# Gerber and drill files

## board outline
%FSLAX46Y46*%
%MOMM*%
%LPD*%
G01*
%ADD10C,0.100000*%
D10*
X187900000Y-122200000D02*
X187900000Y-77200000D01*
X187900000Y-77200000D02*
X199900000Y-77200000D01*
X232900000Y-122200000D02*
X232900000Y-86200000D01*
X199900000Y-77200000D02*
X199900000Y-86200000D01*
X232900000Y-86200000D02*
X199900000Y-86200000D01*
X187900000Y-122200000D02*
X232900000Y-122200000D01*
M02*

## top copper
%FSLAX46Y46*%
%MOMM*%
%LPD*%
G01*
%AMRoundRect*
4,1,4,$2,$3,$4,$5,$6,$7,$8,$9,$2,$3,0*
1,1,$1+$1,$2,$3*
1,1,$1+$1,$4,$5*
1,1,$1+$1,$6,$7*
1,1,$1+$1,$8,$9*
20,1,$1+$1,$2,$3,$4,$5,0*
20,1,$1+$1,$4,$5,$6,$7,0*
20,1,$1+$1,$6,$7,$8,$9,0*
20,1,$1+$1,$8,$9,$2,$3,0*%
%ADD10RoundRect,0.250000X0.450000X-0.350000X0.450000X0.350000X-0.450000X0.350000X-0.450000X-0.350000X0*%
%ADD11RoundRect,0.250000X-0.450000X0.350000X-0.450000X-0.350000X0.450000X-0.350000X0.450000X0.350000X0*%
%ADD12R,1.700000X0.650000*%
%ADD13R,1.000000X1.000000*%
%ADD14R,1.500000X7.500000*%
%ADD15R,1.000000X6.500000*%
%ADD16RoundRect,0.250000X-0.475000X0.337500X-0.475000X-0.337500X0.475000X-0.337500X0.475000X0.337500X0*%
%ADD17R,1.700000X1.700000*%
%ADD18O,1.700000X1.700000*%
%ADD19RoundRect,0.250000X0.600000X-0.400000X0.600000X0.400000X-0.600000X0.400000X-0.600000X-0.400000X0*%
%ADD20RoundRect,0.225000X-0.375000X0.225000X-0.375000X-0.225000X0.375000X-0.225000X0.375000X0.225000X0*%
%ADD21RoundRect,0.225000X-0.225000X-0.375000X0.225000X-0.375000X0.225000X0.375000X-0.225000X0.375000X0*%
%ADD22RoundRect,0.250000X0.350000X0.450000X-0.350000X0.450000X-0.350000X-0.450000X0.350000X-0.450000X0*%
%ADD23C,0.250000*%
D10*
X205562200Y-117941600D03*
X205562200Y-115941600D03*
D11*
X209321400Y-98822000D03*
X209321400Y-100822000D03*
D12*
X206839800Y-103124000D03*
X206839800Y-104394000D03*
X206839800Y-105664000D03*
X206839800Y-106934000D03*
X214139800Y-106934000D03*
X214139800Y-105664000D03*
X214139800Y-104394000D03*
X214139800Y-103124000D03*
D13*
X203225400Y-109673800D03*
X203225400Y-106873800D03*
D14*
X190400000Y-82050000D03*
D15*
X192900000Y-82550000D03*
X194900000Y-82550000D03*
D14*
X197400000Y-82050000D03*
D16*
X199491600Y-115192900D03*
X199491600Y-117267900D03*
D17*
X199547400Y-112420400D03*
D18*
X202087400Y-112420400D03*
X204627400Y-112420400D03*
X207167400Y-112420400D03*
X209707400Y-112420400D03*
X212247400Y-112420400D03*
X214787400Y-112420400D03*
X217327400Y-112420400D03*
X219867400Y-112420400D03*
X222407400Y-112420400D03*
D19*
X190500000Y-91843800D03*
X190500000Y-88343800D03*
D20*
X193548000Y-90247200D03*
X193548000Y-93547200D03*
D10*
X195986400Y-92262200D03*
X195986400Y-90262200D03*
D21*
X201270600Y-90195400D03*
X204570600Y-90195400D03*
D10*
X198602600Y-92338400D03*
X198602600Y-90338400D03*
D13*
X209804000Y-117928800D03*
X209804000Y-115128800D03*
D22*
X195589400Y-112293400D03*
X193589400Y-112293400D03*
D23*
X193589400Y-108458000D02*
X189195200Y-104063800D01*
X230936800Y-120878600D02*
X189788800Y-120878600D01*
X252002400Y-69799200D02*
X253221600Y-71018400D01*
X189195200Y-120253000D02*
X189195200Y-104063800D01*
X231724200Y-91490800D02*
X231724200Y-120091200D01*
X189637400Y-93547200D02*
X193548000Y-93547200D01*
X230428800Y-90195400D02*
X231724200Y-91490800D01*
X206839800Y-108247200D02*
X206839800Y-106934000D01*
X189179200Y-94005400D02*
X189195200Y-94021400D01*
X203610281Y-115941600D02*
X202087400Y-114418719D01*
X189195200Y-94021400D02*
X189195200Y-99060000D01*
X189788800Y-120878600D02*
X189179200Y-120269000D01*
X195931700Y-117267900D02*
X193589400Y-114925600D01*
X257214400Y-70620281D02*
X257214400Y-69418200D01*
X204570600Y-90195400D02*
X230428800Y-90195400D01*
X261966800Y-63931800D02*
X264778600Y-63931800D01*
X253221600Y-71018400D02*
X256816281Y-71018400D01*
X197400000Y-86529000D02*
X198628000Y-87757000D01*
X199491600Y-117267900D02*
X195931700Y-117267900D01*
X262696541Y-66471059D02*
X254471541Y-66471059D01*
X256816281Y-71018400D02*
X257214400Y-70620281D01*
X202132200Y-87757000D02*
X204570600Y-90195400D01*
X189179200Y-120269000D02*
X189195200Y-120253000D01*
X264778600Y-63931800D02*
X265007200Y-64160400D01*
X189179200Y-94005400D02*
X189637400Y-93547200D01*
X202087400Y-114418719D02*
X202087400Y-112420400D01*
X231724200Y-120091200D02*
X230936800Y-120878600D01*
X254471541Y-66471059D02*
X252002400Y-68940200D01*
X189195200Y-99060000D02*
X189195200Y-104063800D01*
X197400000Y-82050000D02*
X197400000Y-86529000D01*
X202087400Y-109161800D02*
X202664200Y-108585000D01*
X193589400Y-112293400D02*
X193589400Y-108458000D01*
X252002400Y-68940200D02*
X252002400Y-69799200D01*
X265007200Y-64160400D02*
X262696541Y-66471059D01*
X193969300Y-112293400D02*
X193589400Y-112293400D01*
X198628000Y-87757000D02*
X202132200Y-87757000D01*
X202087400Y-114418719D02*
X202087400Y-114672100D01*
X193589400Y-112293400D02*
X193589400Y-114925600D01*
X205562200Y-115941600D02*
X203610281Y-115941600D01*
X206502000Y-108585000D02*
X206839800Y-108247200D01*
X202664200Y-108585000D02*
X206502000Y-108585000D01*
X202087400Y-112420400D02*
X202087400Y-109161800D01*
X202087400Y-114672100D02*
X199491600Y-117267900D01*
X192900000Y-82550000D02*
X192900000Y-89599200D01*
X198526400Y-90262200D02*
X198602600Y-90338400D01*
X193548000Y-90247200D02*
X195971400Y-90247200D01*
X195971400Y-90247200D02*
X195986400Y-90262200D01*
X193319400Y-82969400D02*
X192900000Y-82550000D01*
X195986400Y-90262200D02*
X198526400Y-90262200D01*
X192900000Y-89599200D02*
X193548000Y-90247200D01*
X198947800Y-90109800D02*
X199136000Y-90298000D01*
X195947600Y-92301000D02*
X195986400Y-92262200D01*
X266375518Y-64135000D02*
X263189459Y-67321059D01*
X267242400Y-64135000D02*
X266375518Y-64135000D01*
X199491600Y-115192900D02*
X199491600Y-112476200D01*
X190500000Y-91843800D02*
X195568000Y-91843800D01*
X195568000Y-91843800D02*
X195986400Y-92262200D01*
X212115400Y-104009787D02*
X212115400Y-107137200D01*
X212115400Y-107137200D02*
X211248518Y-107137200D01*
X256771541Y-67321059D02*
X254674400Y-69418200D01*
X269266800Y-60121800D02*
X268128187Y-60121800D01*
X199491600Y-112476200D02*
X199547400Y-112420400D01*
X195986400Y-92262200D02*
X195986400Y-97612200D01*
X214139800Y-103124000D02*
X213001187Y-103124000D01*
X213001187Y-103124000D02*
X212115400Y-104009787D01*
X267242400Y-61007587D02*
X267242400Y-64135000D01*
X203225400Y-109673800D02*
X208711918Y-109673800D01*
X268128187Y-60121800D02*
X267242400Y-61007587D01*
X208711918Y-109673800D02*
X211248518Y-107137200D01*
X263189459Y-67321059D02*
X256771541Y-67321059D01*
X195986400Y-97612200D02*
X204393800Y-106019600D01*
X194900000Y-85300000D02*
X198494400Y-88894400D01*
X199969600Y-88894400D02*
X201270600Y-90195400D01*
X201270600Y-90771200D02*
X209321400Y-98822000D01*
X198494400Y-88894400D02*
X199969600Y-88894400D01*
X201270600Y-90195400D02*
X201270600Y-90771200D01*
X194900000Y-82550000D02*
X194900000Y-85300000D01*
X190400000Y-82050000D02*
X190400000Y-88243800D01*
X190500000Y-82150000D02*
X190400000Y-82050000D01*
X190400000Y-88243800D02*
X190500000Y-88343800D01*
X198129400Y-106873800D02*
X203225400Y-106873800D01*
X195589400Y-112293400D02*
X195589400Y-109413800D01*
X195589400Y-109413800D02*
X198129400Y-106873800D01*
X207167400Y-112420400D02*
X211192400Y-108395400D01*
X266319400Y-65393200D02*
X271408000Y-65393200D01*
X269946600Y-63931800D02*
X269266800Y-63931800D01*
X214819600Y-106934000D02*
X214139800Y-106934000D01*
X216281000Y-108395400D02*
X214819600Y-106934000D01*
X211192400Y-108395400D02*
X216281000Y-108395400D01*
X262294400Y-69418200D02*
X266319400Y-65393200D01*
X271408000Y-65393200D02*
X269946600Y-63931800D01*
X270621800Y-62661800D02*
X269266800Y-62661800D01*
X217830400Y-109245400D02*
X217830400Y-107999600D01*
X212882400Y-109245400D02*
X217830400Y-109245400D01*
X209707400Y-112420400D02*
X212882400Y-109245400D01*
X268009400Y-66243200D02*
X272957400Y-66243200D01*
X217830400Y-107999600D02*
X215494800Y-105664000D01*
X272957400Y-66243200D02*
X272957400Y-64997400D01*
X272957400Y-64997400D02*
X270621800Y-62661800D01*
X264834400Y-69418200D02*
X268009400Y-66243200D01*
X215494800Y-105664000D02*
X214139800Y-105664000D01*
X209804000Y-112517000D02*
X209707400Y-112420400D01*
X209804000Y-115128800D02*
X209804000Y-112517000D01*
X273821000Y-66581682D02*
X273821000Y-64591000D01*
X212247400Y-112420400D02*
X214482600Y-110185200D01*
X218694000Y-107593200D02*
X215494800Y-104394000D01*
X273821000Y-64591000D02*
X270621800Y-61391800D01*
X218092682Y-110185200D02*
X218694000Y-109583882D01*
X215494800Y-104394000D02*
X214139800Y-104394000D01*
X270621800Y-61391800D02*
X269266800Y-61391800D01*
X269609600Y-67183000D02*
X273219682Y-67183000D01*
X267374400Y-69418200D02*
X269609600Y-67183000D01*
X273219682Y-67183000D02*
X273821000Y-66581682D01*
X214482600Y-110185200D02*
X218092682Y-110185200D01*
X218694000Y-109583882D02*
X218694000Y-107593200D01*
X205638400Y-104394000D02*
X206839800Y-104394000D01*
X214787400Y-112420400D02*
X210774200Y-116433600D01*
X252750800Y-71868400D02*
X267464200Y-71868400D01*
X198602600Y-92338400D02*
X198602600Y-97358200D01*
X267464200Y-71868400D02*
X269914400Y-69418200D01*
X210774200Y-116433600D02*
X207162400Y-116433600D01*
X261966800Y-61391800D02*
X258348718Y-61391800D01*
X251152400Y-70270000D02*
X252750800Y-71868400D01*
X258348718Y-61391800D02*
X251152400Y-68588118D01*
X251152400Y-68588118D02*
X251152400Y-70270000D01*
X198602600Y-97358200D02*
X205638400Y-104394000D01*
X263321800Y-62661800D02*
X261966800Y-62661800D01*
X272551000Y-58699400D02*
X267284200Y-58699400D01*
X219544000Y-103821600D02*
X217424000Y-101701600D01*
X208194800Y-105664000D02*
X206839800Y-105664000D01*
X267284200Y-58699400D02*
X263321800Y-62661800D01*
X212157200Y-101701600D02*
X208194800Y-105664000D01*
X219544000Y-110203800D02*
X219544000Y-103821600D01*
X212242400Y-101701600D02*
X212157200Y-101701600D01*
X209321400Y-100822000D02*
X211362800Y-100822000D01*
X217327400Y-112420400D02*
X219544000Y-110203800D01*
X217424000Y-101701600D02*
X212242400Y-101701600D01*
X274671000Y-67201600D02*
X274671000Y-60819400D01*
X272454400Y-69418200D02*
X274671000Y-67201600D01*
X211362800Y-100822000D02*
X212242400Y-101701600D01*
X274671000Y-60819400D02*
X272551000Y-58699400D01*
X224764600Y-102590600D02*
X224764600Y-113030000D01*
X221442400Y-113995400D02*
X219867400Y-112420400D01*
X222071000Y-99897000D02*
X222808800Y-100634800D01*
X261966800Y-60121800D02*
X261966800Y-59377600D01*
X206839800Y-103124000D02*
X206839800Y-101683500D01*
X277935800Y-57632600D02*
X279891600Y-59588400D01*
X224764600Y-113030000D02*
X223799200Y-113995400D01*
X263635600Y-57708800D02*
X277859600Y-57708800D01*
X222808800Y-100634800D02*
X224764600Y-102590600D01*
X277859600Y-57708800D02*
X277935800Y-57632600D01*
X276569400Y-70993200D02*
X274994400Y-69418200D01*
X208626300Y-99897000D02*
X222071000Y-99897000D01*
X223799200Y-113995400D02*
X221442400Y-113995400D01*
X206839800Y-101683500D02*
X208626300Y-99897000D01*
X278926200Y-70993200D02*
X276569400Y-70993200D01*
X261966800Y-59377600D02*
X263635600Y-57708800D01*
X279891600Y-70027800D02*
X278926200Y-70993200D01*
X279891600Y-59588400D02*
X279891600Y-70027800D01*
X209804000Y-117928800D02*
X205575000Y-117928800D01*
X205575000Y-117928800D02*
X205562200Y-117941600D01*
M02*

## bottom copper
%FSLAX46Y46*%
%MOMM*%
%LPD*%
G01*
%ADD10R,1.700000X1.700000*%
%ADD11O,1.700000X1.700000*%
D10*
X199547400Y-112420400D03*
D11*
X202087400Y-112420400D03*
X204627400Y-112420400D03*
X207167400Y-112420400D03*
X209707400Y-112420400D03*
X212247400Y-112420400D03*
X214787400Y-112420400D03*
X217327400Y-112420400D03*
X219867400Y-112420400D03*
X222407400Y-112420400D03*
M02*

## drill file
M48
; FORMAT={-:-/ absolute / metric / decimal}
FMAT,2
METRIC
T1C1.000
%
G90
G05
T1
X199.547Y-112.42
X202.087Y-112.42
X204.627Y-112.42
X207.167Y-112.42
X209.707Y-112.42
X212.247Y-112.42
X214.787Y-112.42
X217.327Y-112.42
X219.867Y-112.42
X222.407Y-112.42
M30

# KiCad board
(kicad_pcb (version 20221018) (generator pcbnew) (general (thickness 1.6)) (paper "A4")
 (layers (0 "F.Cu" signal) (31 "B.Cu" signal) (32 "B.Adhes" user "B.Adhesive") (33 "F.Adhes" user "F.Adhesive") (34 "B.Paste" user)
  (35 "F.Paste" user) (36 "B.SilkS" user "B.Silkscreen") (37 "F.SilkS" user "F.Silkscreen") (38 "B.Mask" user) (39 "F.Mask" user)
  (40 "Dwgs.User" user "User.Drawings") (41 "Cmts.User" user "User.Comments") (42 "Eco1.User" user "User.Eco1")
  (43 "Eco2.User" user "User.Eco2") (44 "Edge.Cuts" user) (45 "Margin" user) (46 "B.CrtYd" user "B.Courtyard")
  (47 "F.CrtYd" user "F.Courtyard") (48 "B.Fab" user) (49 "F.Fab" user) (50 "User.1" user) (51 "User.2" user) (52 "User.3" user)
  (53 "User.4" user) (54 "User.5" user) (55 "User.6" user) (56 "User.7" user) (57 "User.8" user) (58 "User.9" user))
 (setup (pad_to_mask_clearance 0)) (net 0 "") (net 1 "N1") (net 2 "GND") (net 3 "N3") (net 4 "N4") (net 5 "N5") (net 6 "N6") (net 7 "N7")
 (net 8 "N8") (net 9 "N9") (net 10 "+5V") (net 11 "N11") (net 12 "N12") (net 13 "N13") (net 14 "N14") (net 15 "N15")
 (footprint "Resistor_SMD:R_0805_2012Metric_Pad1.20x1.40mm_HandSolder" (layer "F.Cu") (at 205.5622 116.9416 90)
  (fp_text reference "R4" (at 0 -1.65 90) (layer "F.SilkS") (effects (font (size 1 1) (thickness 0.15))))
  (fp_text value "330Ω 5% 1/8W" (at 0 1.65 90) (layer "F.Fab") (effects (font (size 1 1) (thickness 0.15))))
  (pad "1" smd roundrect (at -1 0 90) (size 1.2 1.4) (layers "F.Cu" "F.Paste" "F.Mask") (roundrect_rratio 0.208333) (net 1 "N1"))
  (pad "2" smd roundrect (at 1 0 90) (size 1.2 1.4) (layers "F.Cu" "F.Paste" "F.Mask") (roundrect_rratio 0.208333) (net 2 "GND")))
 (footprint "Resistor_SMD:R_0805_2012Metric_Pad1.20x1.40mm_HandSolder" (layer "F.Cu") (at 209.3214 99.822 -90)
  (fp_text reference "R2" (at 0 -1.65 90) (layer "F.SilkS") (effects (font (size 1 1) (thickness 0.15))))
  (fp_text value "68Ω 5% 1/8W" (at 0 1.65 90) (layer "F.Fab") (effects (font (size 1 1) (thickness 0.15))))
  (pad "1" smd roundrect (at -1 0 270) (size 1.2 1.4) (layers "F.Cu" "F.Paste" "F.Mask") (roundrect_rratio 0.208333) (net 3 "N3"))
  (pad "2" smd roundrect (at 1 0 270) (size 1.2 1.4) (layers "F.Cu" "F.Paste" "F.Mask") (roundrect_rratio 0.208333) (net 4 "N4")))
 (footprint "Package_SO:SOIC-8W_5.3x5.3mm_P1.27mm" (layer "F.Cu") (at 210.4898 105.029)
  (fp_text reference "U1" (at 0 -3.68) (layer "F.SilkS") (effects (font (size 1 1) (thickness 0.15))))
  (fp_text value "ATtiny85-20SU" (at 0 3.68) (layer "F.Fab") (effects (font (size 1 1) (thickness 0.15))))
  (pad "1" smd rect (at -3.65 -1.905) (size 1.7 0.65) (layers "F.Cu" "F.Paste" "F.Mask") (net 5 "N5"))
  (pad "2" smd rect (at -3.65 -0.635) (size 1.7 0.65) (layers "F.Cu" "F.Paste" "F.Mask") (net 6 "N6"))
  (pad "3" smd rect (at -3.65 0.635) (size 1.7 0.65) (layers "F.Cu" "F.Paste" "F.Mask") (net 4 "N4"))
  (pad "4" smd rect (at -3.65 1.905) (size 1.7 0.65) (layers "F.Cu" "F.Paste" "F.Mask") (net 2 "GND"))
  (pad "5" smd rect (at 3.65 1.905) (size 1.7 0.65) (layers "F.Cu" "F.Paste" "F.Mask") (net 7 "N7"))
  (pad "6" smd rect (at 3.65 0.635) (size 1.7 0.65) (layers "F.Cu" "F.Paste" "F.Mask") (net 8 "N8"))
  (pad "7" smd rect (at 3.65 -0.635) (size 1.7 0.65) (layers "F.Cu" "F.Paste" "F.Mask") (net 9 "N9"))
  (pad "8" smd rect (at 3.65 -1.905) (size 1.7 0.65) (layers "F.Cu" "F.Paste" "F.Mask") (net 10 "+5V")))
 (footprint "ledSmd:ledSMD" (layer "F.Cu") (at 203.2254 107.8738 90)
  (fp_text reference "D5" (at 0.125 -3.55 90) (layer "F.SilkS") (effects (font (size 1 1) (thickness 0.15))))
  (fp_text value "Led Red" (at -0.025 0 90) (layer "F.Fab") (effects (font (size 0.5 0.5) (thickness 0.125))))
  (pad "1" smd rect (at -1.8 0 90) (size 1 1) (layers "F.Cu" "F.Paste" "F.Mask") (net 10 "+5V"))
  (pad "2" smd rect (at 1 0 90) (size 1 1) (layers "F.Cu" "F.Paste" "F.Mask") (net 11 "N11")))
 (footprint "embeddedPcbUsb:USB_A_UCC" (layer "F.Cu") (at 193.9 82.25 -90)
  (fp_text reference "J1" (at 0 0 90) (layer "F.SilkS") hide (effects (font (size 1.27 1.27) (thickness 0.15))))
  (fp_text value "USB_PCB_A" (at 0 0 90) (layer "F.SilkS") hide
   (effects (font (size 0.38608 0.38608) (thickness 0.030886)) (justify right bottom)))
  (pad "1" smd rect (at -0.2 3.5 270) (size 7.5 1.5) (layers "F.Cu" "F.Paste" "F.Mask") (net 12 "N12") (solder_mask_margin 0.1016))
  (pad "2" smd rect (at 0.3 1 270) (size 6.5 1) (layers "F.Cu" "F.Paste" "F.Mask") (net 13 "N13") (solder_mask_margin 0.1016))
  (pad "3" smd rect (at 0.3 -1 270) (size 6.5 1) (layers "F.Cu" "F.Paste" "F.Mask") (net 3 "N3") (solder_mask_margin 0.1016))
  (pad "4" smd rect (at -0.2 -3.5 270) (size 7.5 1.5) (layers "F.Cu" "F.Paste" "F.Mask") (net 2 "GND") (solder_mask_margin 0.1016)))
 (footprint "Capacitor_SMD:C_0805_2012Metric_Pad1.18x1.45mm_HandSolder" (layer "F.Cu") (at 199.4916 116.2304 -90)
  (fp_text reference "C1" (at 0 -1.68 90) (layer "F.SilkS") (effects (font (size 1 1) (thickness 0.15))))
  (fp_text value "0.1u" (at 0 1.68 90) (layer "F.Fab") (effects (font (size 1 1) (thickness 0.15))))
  (pad "1" smd roundrect (at -1.0375 0 270) (size 1.175 1.45) (layers "F.Cu" "F.Paste" "F.Mask") (roundrect_rratio 0.212766) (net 10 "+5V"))
  (pad "2" smd roundrect (at 1.0375 0 270) (size 1.175 1.45) (layers "F.Cu" "F.Paste" "F.Mask") (roundrect_rratio 0.212766) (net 2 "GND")))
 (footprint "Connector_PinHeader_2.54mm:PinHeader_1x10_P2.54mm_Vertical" (layer "F.Cu") (at 199.5474 112.4204 90)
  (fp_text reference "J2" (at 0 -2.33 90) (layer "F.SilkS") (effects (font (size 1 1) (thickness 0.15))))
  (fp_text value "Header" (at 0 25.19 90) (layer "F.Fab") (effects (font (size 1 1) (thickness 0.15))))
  (pad "1" thru_hole rect (at 0 0 90) (size 1.7 1.7) (drill 1) (layers "*.Cu" "*.Mask") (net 10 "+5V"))
  (pad "2" thru_hole oval (at 0 2.54 90) (size 1.7 1.7) (drill 1) (layers "*.Cu" "*.Mask") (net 2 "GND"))
  (pad "3" thru_hole oval (at 0 5.08 90) (size 1.7 1.7) (drill 1) (layers "*.Cu" "*.Mask") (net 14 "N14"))
  (pad "4" thru_hole oval (at 0 7.62 90) (size 1.7 1.7) (drill 1) (layers "*.Cu" "*.Mask") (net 7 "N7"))
  (pad "5" thru_hole oval (at 0 10.16 90) (size 1.7 1.7) (drill 1) (layers "*.Cu" "*.Mask") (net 8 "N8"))
  (pad "6" thru_hole oval (at 0 12.7 90) (size 1.7 1.7) (drill 1) (layers "*.Cu" "*.Mask") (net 9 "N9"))
  (pad "7" thru_hole oval (at 0 15.24 90) (size 1.7 1.7) (drill 1) (layers "*.Cu" "*.Mask") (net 6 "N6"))
  (pad "8" thru_hole oval (at 0 17.78 90) (size 1.7 1.7) (drill 1) (layers "*.Cu" "*.Mask") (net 4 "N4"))
  (pad "9" thru_hole oval (at 0 20.32 90) (size 1.7 1.7) (drill 1) (layers "*.Cu" "*.Mask") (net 5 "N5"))
  (pad "10" thru_hole oval (at 0 22.86 90) (size 1.7 1.7) (drill 1) (layers "*.Cu" "*.Mask") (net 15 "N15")))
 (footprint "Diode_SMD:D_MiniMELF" (layer "F.Cu") (at 190.5 90.0938 90)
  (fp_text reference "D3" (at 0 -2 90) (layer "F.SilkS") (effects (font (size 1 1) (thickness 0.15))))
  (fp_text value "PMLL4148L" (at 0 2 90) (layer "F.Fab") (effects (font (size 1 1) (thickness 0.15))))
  (pad "1" smd roundrect (at -1.75 0 90) (size 1.3 1.7) (layers "F.Cu" "F.Paste" "F.Mask") (roundrect_rratio 0.1923076923) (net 10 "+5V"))
  (pad "2" smd roundrect (at 1.75 0 90) (size 1.3 1.7) (layers "F.Cu" "F.Paste" "F.Mask") (roundrect_rratio 0.1923076923) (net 12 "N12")))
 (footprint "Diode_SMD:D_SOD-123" (layer "F.Cu") (at 193.548 91.8972 -90)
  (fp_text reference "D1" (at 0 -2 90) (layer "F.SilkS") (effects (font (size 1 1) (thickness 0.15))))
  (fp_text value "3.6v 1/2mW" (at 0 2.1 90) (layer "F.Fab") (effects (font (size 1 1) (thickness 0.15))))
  (pad "1" smd roundrect (at -1.65 0 270) (size 0.9 1.2) (layers "F.Cu" "F.Paste" "F.Mask") (roundrect_rratio 0.25) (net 13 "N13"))
  (pad "2" smd roundrect (at 1.65 0 270) (size 0.9 1.2) (layers "F.Cu" "F.Paste" "F.Mask") (roundrect_rratio 0.25) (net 2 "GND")))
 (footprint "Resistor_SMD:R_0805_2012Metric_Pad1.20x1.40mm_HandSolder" (layer "F.Cu") (at 195.9864 91.2622 90)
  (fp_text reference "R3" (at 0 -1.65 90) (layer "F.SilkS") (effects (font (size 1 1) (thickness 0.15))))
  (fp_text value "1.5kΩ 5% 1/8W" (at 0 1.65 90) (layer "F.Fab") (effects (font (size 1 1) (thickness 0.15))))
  (pad "1" smd roundrect (at -1 0 90) (size 1.2 1.4) (layers "F.Cu" "F.Paste" "F.Mask") (roundrect_rratio 0.208333) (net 10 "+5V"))
  (pad "2" smd roundrect (at 1 0 90) (size 1.2 1.4) (layers "F.Cu" "F.Paste" "F.Mask") (roundrect_rratio 0.208333) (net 13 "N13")))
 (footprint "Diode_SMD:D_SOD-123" (layer "F.Cu") (at 202.9206 90.1954)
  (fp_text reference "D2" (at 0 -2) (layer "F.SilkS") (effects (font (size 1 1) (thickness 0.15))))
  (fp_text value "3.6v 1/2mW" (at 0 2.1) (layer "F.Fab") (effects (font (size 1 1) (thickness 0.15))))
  (pad "1" smd roundrect (at -1.65 0) (size 0.9 1.2) (layers "F.Cu" "F.Paste" "F.Mask") (roundrect_rratio 0.25) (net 3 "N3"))
  (pad "2" smd roundrect (at 1.65 0) (size 0.9 1.2) (layers "F.Cu" "F.Paste" "F.Mask") (roundrect_rratio 0.25) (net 2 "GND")))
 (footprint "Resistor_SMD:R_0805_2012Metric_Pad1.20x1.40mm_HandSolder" (layer "F.Cu") (at 198.6026 91.3384 90)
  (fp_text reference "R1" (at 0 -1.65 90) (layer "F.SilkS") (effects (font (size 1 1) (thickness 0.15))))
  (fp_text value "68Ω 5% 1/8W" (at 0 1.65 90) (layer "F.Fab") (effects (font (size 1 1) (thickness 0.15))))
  (pad "1" smd roundrect (at -1 0 90) (size 1.2 1.4) (layers "F.Cu" "F.Paste" "F.Mask") (roundrect_rratio 0.208333) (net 6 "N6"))
  (pad "2" smd roundrect (at 1 0 90) (size 1.2 1.4) (layers "F.Cu" "F.Paste" "F.Mask") (roundrect_rratio 0.208333) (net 13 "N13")))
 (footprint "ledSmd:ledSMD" (layer "F.Cu") (at 209.804 116.1288 90)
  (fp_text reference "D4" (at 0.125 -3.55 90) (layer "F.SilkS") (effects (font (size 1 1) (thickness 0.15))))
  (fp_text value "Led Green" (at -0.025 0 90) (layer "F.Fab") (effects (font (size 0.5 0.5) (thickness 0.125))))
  (pad "1" smd rect (at -1.8 0 90) (size 1 1) (layers "F.Cu" "F.Paste" "F.Mask") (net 1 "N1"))
  (pad "2" smd rect (at 1 0 90) (size 1 1) (layers "F.Cu" "F.Paste" "F.Mask") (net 8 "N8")))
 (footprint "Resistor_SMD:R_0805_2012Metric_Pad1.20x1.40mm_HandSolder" (layer "F.Cu") (at 194.5894 112.2934 180)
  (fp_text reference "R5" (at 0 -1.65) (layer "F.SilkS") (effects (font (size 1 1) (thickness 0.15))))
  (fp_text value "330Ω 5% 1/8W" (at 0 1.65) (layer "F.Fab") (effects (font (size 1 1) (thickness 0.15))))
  (pad "1" smd roundrect (at -1 0 180) (size 1.2 1.4) (layers "F.Cu" "F.Paste" "F.Mask") (roundrect_rratio 0.208333) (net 11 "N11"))
  (pad "2" smd roundrect (at 1 0 180) (size 1.2 1.4) (layers "F.Cu" "F.Paste" "F.Mask") (roundrect_rratio 0.208333) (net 2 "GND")))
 (gr_line (start 187.9 122.2) (end 187.9 77.2) (stroke (width 0.1) (type default)) (layer "Edge.Cuts"))
 (gr_line (start 187.9 77.2) (end 199.9 77.2) (stroke (width 0.1) (type default)) (layer "Edge.Cuts"))
 (gr_line (start 232.9 122.2) (end 232.9 86.2) (stroke (width 0.1) (type default)) (layer "Edge.Cuts"))
 (gr_line (start 199.9 77.2) (end 199.9 86.2) (stroke (width 0.1) (type default)) (layer "Edge.Cuts"))
 (gr_line (start 232.9 86.2) (end 199.9 86.2) (stroke (width 0.1) (type default)) (layer "Edge.Cuts"))
 (gr_line (start 187.9 122.2) (end 232.9 122.2) (stroke (width 0.1) (type default)) (layer "Edge.Cuts"))
 (segment (start 193.5894 108.458) (end 189.1952 104.0638) (width 0.25) (layer "F.Cu") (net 2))
 (segment (start 230.9368 120.8786) (end 189.7888 120.8786) (width 0.25) (layer "F.Cu") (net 2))
 (segment (start 252.0024 69.7992) (end 253.2216 71.0184) (width 0.25) (layer "F.Cu") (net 2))
 (segment (start 189.1952 120.253) (end 189.1952 104.0638) (width 0.25) (layer "F.Cu") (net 2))
 (segment (start 231.7242 91.4908) (end 231.7242 120.0912) (width 0.25) (layer "F.Cu") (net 2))
 (segment (start 189.6374 93.5472) (end 193.548 93.5472) (width 0.25) (layer "F.Cu") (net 2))
 (segment (start 230.4288 90.1954) (end 231.7242 91.4908) (width 0.25) (layer "F.Cu") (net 2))
 (segment (start 206.8398 108.2472) (end 206.8398 106.934) (width 0.25) (layer "F.Cu") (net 2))
 (segment (start 189.1792 94.0054) (end 189.1952 94.0214) (width 0.25) (layer "F.Cu") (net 2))
 (segment (start 203.610281 115.9416) (end 202.0874 114.418719) (width 0.25) (layer "F.Cu") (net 2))
 (segment (start 189.1952 94.0214) (end 189.1952 99.06) (width 0.25) (layer "F.Cu") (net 2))
 (segment (start 189.7888 120.8786) (end 189.1792 120.269) (width 0.25) (layer "F.Cu") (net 2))
 (segment (start 195.9317 117.2679) (end 193.5894 114.9256) (width 0.25) (layer "F.Cu") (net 2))
 (segment (start 257.2144 70.620281) (end 257.2144 69.4182) (width 0.25) (layer "F.Cu") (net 2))
 (segment (start 204.5706 90.1954) (end 230.4288 90.1954) (width 0.25) (layer "F.Cu") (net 2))
 (segment (start 261.9668 63.9318) (end 264.7786 63.9318) (width 0.25) (layer "F.Cu") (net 2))
 (segment (start 253.2216 71.0184) (end 256.816281 71.0184) (width 0.25) (layer "F.Cu") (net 2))
 (segment (start 197.4 86.529) (end 198.628 87.757) (width 0.25) (layer "F.Cu") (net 2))
 (segment (start 199.4916 117.2679) (end 195.9317 117.2679) (width 0.25) (layer "F.Cu") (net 2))
 (segment (start 262.696541 66.471059) (end 254.471541 66.471059) (width 0.25) (layer "F.Cu") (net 2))
 (segment (start 256.816281 71.0184) (end 257.2144 70.620281) (width 0.25) (layer "F.Cu") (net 2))
 (segment (start 202.1322 87.757) (end 204.5706 90.1954) (width 0.25) (layer "F.Cu") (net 2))
 (segment (start 189.1792 120.269) (end 189.1952 120.253) (width 0.25) (layer "F.Cu") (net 2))
 (segment (start 264.7786 63.9318) (end 265.0072 64.1604) (width 0.25) (layer "F.Cu") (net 2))
 (segment (start 189.1792 94.0054) (end 189.6374 93.5472) (width 0.25) (layer "F.Cu") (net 2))
 (segment (start 202.0874 114.418719) (end 202.0874 112.4204) (width 0.25) (layer "F.Cu") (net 2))
 (segment (start 231.7242 120.0912) (end 230.9368 120.8786) (width 0.25) (layer "F.Cu") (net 2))
 (segment (start 254.471541 66.471059) (end 252.0024 68.9402) (width 0.25) (layer "F.Cu") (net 2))
 (segment (start 189.1952 99.06) (end 189.1952 104.0638) (width 0.25) (layer "F.Cu") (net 2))
 (segment (start 197.4 82.05) (end 197.4 86.529) (width 0.25) (layer "F.Cu") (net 2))
 (segment (start 202.0874 109.1618) (end 202.6642 108.585) (width 0.25) (layer "F.Cu") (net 2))
 (segment (start 193.5894 112.2934) (end 193.5894 108.458) (width 0.25) (layer "F.Cu") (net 2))
 (segment (start 252.0024 68.9402) (end 252.0024 69.7992) (width 0.25) (layer "F.Cu") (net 2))
 (segment (start 265.0072 64.1604) (end 262.696541 66.471059) (width 0.25) (layer "F.Cu") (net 2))
 (segment (start 193.9693 112.2934) (end 193.5894 112.2934) (width 0.25) (layer "F.Cu") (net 2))
 (segment (start 198.628 87.757) (end 202.1322 87.757) (width 0.25) (layer "F.Cu") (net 2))
 (segment (start 202.0874 114.418719) (end 202.0874 114.6721) (width 0.25) (layer "F.Cu") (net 2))
 (segment (start 193.5894 112.2934) (end 193.5894 114.9256) (width 0.25) (layer "F.Cu") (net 2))
 (segment (start 205.5622 115.9416) (end 203.610281 115.9416) (width 0.25) (layer "F.Cu") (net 2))
 (segment (start 206.502 108.585) (end 206.8398 108.2472) (width 0.25) (layer "F.Cu") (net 2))
 (segment (start 202.6642 108.585) (end 206.502 108.585) (width 0.25) (layer "F.Cu") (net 2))
 (segment (start 202.0874 112.4204) (end 202.0874 109.1618) (width 0.25) (layer "F.Cu") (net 2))
 (segment (start 202.0874 114.6721) (end 199.4916 117.2679) (width 0.25) (layer "F.Cu") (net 2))
 (segment (start 192.9 82.55) (end 192.9 89.5992) (width 0.25) (layer "F.Cu") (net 13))
 (segment (start 198.5264 90.2622) (end 198.6026 90.3384) (width 0.25) (layer "F.Cu") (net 13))
 (segment (start 193.548 90.2472) (end 195.9714 90.2472) (width 0.25) (layer "F.Cu") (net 13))
 (segment (start 195.9714 90.2472) (end 195.9864 90.2622) (width 0.25) (layer "F.Cu") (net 13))
 (segment (start 193.3194 82.9694) (end 192.9 82.55) (width 0.25) (layer "F.Cu") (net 13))
 (segment (start 195.9864 90.2622) (end 198.5264 90.2622) (width 0.25) (layer "F.Cu") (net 13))
 (segment (start 192.9 89.5992) (end 193.548 90.2472) (width 0.25) (layer "F.Cu") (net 13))
 (segment (start 198.9478 90.1098) (end 199.136 90.298) (width 0.25) (layer "F.Cu") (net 13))
 (segment (start 195.9476 92.301) (end 195.9864 92.2622) (width 0.25) (layer "F.Cu") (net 10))
 (segment (start 266.375518 64.135) (end 263.189459 67.321059) (width 0.25) (layer "F.Cu") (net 10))
 (segment (start 267.2424 64.135) (end 266.375518 64.135) (width 0.25) (layer "F.Cu") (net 10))
 (segment (start 199.4916 115.1929) (end 199.4916 112.4762) (width 0.25) (layer "F.Cu") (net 10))
 (segment (start 190.5 91.8438) (end 195.568 91.8438) (width 0.25) (layer "F.Cu") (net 10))
 (segment (start 195.568 91.8438) (end 195.9864 92.2622) (width 0.25) (layer "F.Cu") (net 10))
 (segment (start 212.1154 104.009787) (end 212.1154 107.1372) (width 0.25) (layer "F.Cu") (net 10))
 (segment (start 212.1154 107.1372) (end 211.248518 107.1372) (width 0.25) (layer "F.Cu") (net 10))
 (segment (start 256.771541 67.321059) (end 254.6744 69.4182) (width 0.25) (layer "F.Cu") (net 10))
 (segment (start 269.2668 60.1218) (end 268.128187 60.1218) (width 0.25) (layer "F.Cu") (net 10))
 (segment (start 199.4916 112.4762) (end 199.5474 112.4204) (width 0.25) (layer "F.Cu") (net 10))
 (segment (start 195.9864 92.2622) (end 195.9864 97.6122) (width 0.25) (layer "F.Cu") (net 10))
 (segment (start 214.1398 103.124) (end 213.001187 103.124) (width 0.25) (layer "F.Cu") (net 10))
 (segment (start 213.001187 103.124) (end 212.1154 104.009787) (width 0.25) (layer "F.Cu") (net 10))
 (segment (start 267.2424 61.007587) (end 267.2424 64.135) (width 0.25) (layer "F.Cu") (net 10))
 (segment (start 203.2254 109.6738) (end 208.711918 109.6738) (width 0.25) (layer "F.Cu") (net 10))
 (segment (start 268.128187 60.1218) (end 267.2424 61.007587) (width 0.25) (layer "F.Cu") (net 10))
 (segment (start 208.711918 109.6738) (end 211.248518 107.1372) (width 0.25) (layer "F.Cu") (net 10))
 (segment (start 263.189459 67.321059) (end 256.771541 67.321059) (width 0.25) (layer "F.Cu") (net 10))
 (segment (start 195.9864 97.6122) (end 204.3938 106.0196) (width 0.25) (layer "F.Cu") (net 10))
 (segment (start 194.9 85.3) (end 198.4944 88.8944) (width 0.25) (layer "F.Cu") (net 3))
 (segment (start 199.9696 88.8944) (end 201.2706 90.1954) (width 0.25) (layer "F.Cu") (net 3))
 (segment (start 201.2706 90.7712) (end 209.3214 98.822) (width 0.25) (layer "F.Cu") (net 3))
 (segment (start 198.4944 88.8944) (end 199.9696 88.8944) (width 0.25) (layer "F.Cu") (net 3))
 (segment (start 201.2706 90.1954) (end 201.2706 90.7712) (width 0.25) (layer "F.Cu") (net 3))
 (segment (start 194.9 82.55) (end 194.9 85.3) (width 0.25) (layer "F.Cu") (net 3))
 (segment (start 190.4 82.05) (end 190.4 88.2438) (width 0.25) (layer "F.Cu") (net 12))
 (segment (start 190.5 82.15) (end 190.4 82.05) (width 0.25) (layer "F.Cu") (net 12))
 (segment (start 190.4 88.2438) (end 190.5 88.3438) (width 0.25) (layer "F.Cu") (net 12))
 (segment (start 198.1294 106.8738) (end 203.2254 106.8738) (width 0.25) (layer "F.Cu") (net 11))
 (segment (start 195.5894 112.2934) (end 195.5894 109.4138) (width 0.25) (layer "F.Cu") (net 11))
 (segment (start 195.5894 109.4138) (end 198.1294 106.8738) (width 0.25) (layer "F.Cu") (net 11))
 (segment (start 207.1674 112.4204) (end 211.1924 108.3954) (width 0.25) (layer "F.Cu") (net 7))
 (segment (start 266.3194 65.3932) (end 271.408 65.3932) (width 0.25) (layer "F.Cu") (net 7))
 (segment (start 269.9466 63.9318) (end 269.2668 63.9318) (width 0.25) (layer "F.Cu") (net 7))
 (segment (start 214.8196 106.934) (end 214.1398 106.934) (width 0.25) (layer "F.Cu") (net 7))
 (segment (start 216.281 108.3954) (end 214.8196 106.934) (width 0.25) (layer "F.Cu") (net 7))
 (segment (start 211.1924 108.3954) (end 216.281 108.3954) (width 0.25) (layer "F.Cu") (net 7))
 (segment (start 262.2944 69.4182) (end 266.3194 65.3932) (width 0.25) (layer "F.Cu") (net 7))
 (segment (start 271.408 65.3932) (end 269.9466 63.9318) (width 0.25) (layer "F.Cu") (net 7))
 (segment (start 270.6218 62.6618) (end 269.2668 62.6618) (width 0.25) (layer "F.Cu") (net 8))
 (segment (start 217.8304 109.2454) (end 217.8304 107.9996) (width 0.25) (layer "F.Cu") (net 8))
 (segment (start 212.8824 109.2454) (end 217.8304 109.2454) (width 0.25) (layer "F.Cu") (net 8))
 (segment (start 209.7074 112.4204) (end 212.8824 109.2454) (width 0.25) (layer "F.Cu") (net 8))
 (segment (start 268.0094 66.2432) (end 272.9574 66.2432) (width 0.25) (layer "F.Cu") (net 8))
 (segment (start 217.8304 107.9996) (end 215.4948 105.664) (width 0.25) (layer "F.Cu") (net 8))
 (segment (start 272.9574 66.2432) (end 272.9574 64.9974) (width 0.25) (layer "F.Cu") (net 8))
 (segment (start 272.9574 64.9974) (end 270.6218 62.6618) (width 0.25) (layer "F.Cu") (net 8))
 (segment (start 264.8344 69.4182) (end 268.0094 66.2432) (width 0.25) (layer "F.Cu") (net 8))
 (segment (start 215.4948 105.664) (end 214.1398 105.664) (width 0.25) (layer "F.Cu") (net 8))
 (segment (start 209.804 112.517) (end 209.7074 112.4204) (width 0.25) (layer "F.Cu") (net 8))
 (segment (start 209.804 115.1288) (end 209.804 112.517) (width 0.25) (layer "F.Cu") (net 8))
 (segment (start 273.821 66.581682) (end 273.821 64.591) (width 0.25) (layer "F.Cu") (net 9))
 (segment (start 212.2474 112.4204) (end 214.4826 110.1852) (width 0.25) (layer "F.Cu") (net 9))
 (segment (start 218.694 107.5932) (end 215.4948 104.394) (width 0.25) (layer "F.Cu") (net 9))
 (segment (start 273.821 64.591) (end 270.6218 61.3918) (width 0.25) (layer "F.Cu") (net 9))
 (segment (start 218.092682 110.1852) (end 218.694 109.583882) (width 0.25) (layer "F.Cu") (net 9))
 (segment (start 215.4948 104.394) (end 214.1398 104.394) (width 0.25) (layer "F.Cu") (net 9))
 (segment (start 270.6218 61.3918) (end 269.2668 61.3918) (width 0.25) (layer "F.Cu") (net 9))
 (segment (start 269.6096 67.183) (end 273.219682 67.183) (width 0.25) (layer "F.Cu") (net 9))
 (segment (start 267.3744 69.4182) (end 269.6096 67.183) (width 0.25) (layer "F.Cu") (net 9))
 (segment (start 273.219682 67.183) (end 273.821 66.581682) (width 0.25) (layer "F.Cu") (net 9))
 (segment (start 214.4826 110.1852) (end 218.092682 110.1852) (width 0.25) (layer "F.Cu") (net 9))
 (segment (start 218.694 109.583882) (end 218.694 107.5932) (width 0.25) (layer "F.Cu") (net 9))
 (segment (start 205.6384 104.394) (end 206.8398 104.394) (width 0.25) (layer "F.Cu") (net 6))
 (segment (start 214.7874 112.4204) (end 210.7742 116.4336) (width 0.25) (layer "F.Cu") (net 6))
 (segment (start 252.7508 71.8684) (end 267.4642 71.8684) (width 0.25) (layer "F.Cu") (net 6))
 (segment (start 198.6026 92.3384) (end 198.6026 97.3582) (width 0.25) (layer "F.Cu") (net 6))
 (segment (start 267.4642 71.8684) (end 269.9144 69.4182) (width 0.25) (layer "F.Cu") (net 6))
 (segment (start 210.7742 116.4336) (end 207.1624 116.4336) (width 0.25) (layer "F.Cu") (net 6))
 (segment (start 261.9668 61.3918) (end 258.348718 61.3918) (width 0.25) (layer "F.Cu") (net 6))
 (segment (start 251.1524 70.27) (end 252.7508 71.8684) (width 0.25) (layer "F.Cu") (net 6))
 (segment (start 258.348718 61.3918) (end 251.1524 68.588118) (width 0.25) (layer "F.Cu") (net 6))
 (segment (start 251.1524 68.588118) (end 251.1524 70.27) (width 0.25) (layer "F.Cu") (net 6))
 (segment (start 198.6026 97.3582) (end 205.6384 104.394) (width 0.25) (layer "F.Cu") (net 6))
 (segment (start 263.3218 62.6618) (end 261.9668 62.6618) (width 0.25) (layer "F.Cu") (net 4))
 (segment (start 272.551 58.6994) (end 267.2842 58.6994) (width 0.25) (layer "F.Cu") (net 4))
 (segment (start 219.544 103.8216) (end 217.424 101.7016) (width 0.25) (layer "F.Cu") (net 4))
 (segment (start 208.1948 105.664) (end 206.8398 105.664) (width 0.25) (layer "F.Cu") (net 4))
 (segment (start 267.2842 58.6994) (end 263.3218 62.6618) (width 0.25) (layer "F.Cu") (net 4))
 (segment (start 212.1572 101.7016) (end 208.1948 105.664) (width 0.25) (layer "F.Cu") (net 4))
 (segment (start 219.544 110.2038) (end 219.544 103.8216) (width 0.25) (layer "F.Cu") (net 4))
 (segment (start 212.2424 101.7016) (end 212.1572 101.7016) (width 0.25) (layer "F.Cu") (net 4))
 (segment (start 209.3214 100.822) (end 211.3628 100.822) (width 0.25) (layer "F.Cu") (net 4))
 (segment (start 217.3274 112.4204) (end 219.544 110.2038) (width 0.25) (layer "F.Cu") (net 4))
 (segment (start 217.424 101.7016) (end 212.2424 101.7016) (width 0.25) (layer "F.Cu") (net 4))
 (segment (start 274.671 67.2016) (end 274.671 60.8194) (width 0.25) (layer "F.Cu") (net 4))
 (segment (start 272.4544 69.4182) (end 274.671 67.2016) (width 0.25) (layer "F.Cu") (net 4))
 (segment (start 211.3628 100.822) (end 212.2424 101.7016) (width 0.25) (layer "F.Cu") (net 4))
 (segment (start 274.671 60.8194) (end 272.551 58.6994) (width 0.25) (layer "F.Cu") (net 4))
 (segment (start 224.7646 102.5906) (end 224.7646 113.03) (width 0.25) (layer "F.Cu") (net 5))
 (segment (start 221.4424 113.9954) (end 219.8674 112.4204) (width 0.25) (layer "F.Cu") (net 5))
 (segment (start 222.071 99.897) (end 222.8088 100.6348) (width 0.25) (layer "F.Cu") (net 5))
 (segment (start 261.9668 60.1218) (end 261.9668 59.3776) (width 0.25) (layer "F.Cu") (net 5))
 (segment (start 206.8398 103.124) (end 206.8398 101.6835) (width 0.25) (layer "F.Cu") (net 5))
 (segment (start 277.9358 57.6326) (end 279.8916 59.5884) (width 0.25) (layer "F.Cu") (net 5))
 (segment (start 224.7646 113.03) (end 223.7992 113.9954) (width 0.25) (layer "F.Cu") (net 5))
 (segment (start 263.6356 57.7088) (end 277.8596 57.7088) (width 0.25) (layer "F.Cu") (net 5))
 (segment (start 222.8088 100.6348) (end 224.7646 102.5906) (width 0.25) (layer "F.Cu") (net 5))
 (segment (start 277.8596 57.7088) (end 277.9358 57.6326) (width 0.25) (layer "F.Cu") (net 5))
 (segment (start 276.5694 70.9932) (end 274.9944 69.4182) (width 0.25) (layer "F.Cu") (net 5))
 (segment (start 208.6263 99.897) (end 222.071 99.897) (width 0.25) (layer "F.Cu") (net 5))
 (segment (start 223.7992 113.9954) (end 221.4424 113.9954) (width 0.25) (layer "F.Cu") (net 5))
 (segment (start 206.8398 101.6835) (end 208.6263 99.897) (width 0.25) (layer "F.Cu") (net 5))
 (segment (start 278.9262 70.9932) (end 276.5694 70.9932) (width 0.25) (layer "F.Cu") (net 5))
 (segment (start 261.9668 59.3776) (end 263.6356 57.7088) (width 0.25) (layer "F.Cu") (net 5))
 (segment (start 279.8916 70.0278) (end 278.9262 70.9932) (width 0.25) (layer "F.Cu") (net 5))
 (segment (start 279.8916 59.5884) (end 279.8916 70.0278) (width 0.25) (layer "F.Cu") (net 5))
 (segment (start 209.804 117.9288) (end 205.575 117.9288) (width 0.25) (layer "F.Cu") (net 1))
 (segment (start 205.575 117.9288) (end 205.5622 117.9416) (width 0.25) (layer "F.Cu") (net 1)))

